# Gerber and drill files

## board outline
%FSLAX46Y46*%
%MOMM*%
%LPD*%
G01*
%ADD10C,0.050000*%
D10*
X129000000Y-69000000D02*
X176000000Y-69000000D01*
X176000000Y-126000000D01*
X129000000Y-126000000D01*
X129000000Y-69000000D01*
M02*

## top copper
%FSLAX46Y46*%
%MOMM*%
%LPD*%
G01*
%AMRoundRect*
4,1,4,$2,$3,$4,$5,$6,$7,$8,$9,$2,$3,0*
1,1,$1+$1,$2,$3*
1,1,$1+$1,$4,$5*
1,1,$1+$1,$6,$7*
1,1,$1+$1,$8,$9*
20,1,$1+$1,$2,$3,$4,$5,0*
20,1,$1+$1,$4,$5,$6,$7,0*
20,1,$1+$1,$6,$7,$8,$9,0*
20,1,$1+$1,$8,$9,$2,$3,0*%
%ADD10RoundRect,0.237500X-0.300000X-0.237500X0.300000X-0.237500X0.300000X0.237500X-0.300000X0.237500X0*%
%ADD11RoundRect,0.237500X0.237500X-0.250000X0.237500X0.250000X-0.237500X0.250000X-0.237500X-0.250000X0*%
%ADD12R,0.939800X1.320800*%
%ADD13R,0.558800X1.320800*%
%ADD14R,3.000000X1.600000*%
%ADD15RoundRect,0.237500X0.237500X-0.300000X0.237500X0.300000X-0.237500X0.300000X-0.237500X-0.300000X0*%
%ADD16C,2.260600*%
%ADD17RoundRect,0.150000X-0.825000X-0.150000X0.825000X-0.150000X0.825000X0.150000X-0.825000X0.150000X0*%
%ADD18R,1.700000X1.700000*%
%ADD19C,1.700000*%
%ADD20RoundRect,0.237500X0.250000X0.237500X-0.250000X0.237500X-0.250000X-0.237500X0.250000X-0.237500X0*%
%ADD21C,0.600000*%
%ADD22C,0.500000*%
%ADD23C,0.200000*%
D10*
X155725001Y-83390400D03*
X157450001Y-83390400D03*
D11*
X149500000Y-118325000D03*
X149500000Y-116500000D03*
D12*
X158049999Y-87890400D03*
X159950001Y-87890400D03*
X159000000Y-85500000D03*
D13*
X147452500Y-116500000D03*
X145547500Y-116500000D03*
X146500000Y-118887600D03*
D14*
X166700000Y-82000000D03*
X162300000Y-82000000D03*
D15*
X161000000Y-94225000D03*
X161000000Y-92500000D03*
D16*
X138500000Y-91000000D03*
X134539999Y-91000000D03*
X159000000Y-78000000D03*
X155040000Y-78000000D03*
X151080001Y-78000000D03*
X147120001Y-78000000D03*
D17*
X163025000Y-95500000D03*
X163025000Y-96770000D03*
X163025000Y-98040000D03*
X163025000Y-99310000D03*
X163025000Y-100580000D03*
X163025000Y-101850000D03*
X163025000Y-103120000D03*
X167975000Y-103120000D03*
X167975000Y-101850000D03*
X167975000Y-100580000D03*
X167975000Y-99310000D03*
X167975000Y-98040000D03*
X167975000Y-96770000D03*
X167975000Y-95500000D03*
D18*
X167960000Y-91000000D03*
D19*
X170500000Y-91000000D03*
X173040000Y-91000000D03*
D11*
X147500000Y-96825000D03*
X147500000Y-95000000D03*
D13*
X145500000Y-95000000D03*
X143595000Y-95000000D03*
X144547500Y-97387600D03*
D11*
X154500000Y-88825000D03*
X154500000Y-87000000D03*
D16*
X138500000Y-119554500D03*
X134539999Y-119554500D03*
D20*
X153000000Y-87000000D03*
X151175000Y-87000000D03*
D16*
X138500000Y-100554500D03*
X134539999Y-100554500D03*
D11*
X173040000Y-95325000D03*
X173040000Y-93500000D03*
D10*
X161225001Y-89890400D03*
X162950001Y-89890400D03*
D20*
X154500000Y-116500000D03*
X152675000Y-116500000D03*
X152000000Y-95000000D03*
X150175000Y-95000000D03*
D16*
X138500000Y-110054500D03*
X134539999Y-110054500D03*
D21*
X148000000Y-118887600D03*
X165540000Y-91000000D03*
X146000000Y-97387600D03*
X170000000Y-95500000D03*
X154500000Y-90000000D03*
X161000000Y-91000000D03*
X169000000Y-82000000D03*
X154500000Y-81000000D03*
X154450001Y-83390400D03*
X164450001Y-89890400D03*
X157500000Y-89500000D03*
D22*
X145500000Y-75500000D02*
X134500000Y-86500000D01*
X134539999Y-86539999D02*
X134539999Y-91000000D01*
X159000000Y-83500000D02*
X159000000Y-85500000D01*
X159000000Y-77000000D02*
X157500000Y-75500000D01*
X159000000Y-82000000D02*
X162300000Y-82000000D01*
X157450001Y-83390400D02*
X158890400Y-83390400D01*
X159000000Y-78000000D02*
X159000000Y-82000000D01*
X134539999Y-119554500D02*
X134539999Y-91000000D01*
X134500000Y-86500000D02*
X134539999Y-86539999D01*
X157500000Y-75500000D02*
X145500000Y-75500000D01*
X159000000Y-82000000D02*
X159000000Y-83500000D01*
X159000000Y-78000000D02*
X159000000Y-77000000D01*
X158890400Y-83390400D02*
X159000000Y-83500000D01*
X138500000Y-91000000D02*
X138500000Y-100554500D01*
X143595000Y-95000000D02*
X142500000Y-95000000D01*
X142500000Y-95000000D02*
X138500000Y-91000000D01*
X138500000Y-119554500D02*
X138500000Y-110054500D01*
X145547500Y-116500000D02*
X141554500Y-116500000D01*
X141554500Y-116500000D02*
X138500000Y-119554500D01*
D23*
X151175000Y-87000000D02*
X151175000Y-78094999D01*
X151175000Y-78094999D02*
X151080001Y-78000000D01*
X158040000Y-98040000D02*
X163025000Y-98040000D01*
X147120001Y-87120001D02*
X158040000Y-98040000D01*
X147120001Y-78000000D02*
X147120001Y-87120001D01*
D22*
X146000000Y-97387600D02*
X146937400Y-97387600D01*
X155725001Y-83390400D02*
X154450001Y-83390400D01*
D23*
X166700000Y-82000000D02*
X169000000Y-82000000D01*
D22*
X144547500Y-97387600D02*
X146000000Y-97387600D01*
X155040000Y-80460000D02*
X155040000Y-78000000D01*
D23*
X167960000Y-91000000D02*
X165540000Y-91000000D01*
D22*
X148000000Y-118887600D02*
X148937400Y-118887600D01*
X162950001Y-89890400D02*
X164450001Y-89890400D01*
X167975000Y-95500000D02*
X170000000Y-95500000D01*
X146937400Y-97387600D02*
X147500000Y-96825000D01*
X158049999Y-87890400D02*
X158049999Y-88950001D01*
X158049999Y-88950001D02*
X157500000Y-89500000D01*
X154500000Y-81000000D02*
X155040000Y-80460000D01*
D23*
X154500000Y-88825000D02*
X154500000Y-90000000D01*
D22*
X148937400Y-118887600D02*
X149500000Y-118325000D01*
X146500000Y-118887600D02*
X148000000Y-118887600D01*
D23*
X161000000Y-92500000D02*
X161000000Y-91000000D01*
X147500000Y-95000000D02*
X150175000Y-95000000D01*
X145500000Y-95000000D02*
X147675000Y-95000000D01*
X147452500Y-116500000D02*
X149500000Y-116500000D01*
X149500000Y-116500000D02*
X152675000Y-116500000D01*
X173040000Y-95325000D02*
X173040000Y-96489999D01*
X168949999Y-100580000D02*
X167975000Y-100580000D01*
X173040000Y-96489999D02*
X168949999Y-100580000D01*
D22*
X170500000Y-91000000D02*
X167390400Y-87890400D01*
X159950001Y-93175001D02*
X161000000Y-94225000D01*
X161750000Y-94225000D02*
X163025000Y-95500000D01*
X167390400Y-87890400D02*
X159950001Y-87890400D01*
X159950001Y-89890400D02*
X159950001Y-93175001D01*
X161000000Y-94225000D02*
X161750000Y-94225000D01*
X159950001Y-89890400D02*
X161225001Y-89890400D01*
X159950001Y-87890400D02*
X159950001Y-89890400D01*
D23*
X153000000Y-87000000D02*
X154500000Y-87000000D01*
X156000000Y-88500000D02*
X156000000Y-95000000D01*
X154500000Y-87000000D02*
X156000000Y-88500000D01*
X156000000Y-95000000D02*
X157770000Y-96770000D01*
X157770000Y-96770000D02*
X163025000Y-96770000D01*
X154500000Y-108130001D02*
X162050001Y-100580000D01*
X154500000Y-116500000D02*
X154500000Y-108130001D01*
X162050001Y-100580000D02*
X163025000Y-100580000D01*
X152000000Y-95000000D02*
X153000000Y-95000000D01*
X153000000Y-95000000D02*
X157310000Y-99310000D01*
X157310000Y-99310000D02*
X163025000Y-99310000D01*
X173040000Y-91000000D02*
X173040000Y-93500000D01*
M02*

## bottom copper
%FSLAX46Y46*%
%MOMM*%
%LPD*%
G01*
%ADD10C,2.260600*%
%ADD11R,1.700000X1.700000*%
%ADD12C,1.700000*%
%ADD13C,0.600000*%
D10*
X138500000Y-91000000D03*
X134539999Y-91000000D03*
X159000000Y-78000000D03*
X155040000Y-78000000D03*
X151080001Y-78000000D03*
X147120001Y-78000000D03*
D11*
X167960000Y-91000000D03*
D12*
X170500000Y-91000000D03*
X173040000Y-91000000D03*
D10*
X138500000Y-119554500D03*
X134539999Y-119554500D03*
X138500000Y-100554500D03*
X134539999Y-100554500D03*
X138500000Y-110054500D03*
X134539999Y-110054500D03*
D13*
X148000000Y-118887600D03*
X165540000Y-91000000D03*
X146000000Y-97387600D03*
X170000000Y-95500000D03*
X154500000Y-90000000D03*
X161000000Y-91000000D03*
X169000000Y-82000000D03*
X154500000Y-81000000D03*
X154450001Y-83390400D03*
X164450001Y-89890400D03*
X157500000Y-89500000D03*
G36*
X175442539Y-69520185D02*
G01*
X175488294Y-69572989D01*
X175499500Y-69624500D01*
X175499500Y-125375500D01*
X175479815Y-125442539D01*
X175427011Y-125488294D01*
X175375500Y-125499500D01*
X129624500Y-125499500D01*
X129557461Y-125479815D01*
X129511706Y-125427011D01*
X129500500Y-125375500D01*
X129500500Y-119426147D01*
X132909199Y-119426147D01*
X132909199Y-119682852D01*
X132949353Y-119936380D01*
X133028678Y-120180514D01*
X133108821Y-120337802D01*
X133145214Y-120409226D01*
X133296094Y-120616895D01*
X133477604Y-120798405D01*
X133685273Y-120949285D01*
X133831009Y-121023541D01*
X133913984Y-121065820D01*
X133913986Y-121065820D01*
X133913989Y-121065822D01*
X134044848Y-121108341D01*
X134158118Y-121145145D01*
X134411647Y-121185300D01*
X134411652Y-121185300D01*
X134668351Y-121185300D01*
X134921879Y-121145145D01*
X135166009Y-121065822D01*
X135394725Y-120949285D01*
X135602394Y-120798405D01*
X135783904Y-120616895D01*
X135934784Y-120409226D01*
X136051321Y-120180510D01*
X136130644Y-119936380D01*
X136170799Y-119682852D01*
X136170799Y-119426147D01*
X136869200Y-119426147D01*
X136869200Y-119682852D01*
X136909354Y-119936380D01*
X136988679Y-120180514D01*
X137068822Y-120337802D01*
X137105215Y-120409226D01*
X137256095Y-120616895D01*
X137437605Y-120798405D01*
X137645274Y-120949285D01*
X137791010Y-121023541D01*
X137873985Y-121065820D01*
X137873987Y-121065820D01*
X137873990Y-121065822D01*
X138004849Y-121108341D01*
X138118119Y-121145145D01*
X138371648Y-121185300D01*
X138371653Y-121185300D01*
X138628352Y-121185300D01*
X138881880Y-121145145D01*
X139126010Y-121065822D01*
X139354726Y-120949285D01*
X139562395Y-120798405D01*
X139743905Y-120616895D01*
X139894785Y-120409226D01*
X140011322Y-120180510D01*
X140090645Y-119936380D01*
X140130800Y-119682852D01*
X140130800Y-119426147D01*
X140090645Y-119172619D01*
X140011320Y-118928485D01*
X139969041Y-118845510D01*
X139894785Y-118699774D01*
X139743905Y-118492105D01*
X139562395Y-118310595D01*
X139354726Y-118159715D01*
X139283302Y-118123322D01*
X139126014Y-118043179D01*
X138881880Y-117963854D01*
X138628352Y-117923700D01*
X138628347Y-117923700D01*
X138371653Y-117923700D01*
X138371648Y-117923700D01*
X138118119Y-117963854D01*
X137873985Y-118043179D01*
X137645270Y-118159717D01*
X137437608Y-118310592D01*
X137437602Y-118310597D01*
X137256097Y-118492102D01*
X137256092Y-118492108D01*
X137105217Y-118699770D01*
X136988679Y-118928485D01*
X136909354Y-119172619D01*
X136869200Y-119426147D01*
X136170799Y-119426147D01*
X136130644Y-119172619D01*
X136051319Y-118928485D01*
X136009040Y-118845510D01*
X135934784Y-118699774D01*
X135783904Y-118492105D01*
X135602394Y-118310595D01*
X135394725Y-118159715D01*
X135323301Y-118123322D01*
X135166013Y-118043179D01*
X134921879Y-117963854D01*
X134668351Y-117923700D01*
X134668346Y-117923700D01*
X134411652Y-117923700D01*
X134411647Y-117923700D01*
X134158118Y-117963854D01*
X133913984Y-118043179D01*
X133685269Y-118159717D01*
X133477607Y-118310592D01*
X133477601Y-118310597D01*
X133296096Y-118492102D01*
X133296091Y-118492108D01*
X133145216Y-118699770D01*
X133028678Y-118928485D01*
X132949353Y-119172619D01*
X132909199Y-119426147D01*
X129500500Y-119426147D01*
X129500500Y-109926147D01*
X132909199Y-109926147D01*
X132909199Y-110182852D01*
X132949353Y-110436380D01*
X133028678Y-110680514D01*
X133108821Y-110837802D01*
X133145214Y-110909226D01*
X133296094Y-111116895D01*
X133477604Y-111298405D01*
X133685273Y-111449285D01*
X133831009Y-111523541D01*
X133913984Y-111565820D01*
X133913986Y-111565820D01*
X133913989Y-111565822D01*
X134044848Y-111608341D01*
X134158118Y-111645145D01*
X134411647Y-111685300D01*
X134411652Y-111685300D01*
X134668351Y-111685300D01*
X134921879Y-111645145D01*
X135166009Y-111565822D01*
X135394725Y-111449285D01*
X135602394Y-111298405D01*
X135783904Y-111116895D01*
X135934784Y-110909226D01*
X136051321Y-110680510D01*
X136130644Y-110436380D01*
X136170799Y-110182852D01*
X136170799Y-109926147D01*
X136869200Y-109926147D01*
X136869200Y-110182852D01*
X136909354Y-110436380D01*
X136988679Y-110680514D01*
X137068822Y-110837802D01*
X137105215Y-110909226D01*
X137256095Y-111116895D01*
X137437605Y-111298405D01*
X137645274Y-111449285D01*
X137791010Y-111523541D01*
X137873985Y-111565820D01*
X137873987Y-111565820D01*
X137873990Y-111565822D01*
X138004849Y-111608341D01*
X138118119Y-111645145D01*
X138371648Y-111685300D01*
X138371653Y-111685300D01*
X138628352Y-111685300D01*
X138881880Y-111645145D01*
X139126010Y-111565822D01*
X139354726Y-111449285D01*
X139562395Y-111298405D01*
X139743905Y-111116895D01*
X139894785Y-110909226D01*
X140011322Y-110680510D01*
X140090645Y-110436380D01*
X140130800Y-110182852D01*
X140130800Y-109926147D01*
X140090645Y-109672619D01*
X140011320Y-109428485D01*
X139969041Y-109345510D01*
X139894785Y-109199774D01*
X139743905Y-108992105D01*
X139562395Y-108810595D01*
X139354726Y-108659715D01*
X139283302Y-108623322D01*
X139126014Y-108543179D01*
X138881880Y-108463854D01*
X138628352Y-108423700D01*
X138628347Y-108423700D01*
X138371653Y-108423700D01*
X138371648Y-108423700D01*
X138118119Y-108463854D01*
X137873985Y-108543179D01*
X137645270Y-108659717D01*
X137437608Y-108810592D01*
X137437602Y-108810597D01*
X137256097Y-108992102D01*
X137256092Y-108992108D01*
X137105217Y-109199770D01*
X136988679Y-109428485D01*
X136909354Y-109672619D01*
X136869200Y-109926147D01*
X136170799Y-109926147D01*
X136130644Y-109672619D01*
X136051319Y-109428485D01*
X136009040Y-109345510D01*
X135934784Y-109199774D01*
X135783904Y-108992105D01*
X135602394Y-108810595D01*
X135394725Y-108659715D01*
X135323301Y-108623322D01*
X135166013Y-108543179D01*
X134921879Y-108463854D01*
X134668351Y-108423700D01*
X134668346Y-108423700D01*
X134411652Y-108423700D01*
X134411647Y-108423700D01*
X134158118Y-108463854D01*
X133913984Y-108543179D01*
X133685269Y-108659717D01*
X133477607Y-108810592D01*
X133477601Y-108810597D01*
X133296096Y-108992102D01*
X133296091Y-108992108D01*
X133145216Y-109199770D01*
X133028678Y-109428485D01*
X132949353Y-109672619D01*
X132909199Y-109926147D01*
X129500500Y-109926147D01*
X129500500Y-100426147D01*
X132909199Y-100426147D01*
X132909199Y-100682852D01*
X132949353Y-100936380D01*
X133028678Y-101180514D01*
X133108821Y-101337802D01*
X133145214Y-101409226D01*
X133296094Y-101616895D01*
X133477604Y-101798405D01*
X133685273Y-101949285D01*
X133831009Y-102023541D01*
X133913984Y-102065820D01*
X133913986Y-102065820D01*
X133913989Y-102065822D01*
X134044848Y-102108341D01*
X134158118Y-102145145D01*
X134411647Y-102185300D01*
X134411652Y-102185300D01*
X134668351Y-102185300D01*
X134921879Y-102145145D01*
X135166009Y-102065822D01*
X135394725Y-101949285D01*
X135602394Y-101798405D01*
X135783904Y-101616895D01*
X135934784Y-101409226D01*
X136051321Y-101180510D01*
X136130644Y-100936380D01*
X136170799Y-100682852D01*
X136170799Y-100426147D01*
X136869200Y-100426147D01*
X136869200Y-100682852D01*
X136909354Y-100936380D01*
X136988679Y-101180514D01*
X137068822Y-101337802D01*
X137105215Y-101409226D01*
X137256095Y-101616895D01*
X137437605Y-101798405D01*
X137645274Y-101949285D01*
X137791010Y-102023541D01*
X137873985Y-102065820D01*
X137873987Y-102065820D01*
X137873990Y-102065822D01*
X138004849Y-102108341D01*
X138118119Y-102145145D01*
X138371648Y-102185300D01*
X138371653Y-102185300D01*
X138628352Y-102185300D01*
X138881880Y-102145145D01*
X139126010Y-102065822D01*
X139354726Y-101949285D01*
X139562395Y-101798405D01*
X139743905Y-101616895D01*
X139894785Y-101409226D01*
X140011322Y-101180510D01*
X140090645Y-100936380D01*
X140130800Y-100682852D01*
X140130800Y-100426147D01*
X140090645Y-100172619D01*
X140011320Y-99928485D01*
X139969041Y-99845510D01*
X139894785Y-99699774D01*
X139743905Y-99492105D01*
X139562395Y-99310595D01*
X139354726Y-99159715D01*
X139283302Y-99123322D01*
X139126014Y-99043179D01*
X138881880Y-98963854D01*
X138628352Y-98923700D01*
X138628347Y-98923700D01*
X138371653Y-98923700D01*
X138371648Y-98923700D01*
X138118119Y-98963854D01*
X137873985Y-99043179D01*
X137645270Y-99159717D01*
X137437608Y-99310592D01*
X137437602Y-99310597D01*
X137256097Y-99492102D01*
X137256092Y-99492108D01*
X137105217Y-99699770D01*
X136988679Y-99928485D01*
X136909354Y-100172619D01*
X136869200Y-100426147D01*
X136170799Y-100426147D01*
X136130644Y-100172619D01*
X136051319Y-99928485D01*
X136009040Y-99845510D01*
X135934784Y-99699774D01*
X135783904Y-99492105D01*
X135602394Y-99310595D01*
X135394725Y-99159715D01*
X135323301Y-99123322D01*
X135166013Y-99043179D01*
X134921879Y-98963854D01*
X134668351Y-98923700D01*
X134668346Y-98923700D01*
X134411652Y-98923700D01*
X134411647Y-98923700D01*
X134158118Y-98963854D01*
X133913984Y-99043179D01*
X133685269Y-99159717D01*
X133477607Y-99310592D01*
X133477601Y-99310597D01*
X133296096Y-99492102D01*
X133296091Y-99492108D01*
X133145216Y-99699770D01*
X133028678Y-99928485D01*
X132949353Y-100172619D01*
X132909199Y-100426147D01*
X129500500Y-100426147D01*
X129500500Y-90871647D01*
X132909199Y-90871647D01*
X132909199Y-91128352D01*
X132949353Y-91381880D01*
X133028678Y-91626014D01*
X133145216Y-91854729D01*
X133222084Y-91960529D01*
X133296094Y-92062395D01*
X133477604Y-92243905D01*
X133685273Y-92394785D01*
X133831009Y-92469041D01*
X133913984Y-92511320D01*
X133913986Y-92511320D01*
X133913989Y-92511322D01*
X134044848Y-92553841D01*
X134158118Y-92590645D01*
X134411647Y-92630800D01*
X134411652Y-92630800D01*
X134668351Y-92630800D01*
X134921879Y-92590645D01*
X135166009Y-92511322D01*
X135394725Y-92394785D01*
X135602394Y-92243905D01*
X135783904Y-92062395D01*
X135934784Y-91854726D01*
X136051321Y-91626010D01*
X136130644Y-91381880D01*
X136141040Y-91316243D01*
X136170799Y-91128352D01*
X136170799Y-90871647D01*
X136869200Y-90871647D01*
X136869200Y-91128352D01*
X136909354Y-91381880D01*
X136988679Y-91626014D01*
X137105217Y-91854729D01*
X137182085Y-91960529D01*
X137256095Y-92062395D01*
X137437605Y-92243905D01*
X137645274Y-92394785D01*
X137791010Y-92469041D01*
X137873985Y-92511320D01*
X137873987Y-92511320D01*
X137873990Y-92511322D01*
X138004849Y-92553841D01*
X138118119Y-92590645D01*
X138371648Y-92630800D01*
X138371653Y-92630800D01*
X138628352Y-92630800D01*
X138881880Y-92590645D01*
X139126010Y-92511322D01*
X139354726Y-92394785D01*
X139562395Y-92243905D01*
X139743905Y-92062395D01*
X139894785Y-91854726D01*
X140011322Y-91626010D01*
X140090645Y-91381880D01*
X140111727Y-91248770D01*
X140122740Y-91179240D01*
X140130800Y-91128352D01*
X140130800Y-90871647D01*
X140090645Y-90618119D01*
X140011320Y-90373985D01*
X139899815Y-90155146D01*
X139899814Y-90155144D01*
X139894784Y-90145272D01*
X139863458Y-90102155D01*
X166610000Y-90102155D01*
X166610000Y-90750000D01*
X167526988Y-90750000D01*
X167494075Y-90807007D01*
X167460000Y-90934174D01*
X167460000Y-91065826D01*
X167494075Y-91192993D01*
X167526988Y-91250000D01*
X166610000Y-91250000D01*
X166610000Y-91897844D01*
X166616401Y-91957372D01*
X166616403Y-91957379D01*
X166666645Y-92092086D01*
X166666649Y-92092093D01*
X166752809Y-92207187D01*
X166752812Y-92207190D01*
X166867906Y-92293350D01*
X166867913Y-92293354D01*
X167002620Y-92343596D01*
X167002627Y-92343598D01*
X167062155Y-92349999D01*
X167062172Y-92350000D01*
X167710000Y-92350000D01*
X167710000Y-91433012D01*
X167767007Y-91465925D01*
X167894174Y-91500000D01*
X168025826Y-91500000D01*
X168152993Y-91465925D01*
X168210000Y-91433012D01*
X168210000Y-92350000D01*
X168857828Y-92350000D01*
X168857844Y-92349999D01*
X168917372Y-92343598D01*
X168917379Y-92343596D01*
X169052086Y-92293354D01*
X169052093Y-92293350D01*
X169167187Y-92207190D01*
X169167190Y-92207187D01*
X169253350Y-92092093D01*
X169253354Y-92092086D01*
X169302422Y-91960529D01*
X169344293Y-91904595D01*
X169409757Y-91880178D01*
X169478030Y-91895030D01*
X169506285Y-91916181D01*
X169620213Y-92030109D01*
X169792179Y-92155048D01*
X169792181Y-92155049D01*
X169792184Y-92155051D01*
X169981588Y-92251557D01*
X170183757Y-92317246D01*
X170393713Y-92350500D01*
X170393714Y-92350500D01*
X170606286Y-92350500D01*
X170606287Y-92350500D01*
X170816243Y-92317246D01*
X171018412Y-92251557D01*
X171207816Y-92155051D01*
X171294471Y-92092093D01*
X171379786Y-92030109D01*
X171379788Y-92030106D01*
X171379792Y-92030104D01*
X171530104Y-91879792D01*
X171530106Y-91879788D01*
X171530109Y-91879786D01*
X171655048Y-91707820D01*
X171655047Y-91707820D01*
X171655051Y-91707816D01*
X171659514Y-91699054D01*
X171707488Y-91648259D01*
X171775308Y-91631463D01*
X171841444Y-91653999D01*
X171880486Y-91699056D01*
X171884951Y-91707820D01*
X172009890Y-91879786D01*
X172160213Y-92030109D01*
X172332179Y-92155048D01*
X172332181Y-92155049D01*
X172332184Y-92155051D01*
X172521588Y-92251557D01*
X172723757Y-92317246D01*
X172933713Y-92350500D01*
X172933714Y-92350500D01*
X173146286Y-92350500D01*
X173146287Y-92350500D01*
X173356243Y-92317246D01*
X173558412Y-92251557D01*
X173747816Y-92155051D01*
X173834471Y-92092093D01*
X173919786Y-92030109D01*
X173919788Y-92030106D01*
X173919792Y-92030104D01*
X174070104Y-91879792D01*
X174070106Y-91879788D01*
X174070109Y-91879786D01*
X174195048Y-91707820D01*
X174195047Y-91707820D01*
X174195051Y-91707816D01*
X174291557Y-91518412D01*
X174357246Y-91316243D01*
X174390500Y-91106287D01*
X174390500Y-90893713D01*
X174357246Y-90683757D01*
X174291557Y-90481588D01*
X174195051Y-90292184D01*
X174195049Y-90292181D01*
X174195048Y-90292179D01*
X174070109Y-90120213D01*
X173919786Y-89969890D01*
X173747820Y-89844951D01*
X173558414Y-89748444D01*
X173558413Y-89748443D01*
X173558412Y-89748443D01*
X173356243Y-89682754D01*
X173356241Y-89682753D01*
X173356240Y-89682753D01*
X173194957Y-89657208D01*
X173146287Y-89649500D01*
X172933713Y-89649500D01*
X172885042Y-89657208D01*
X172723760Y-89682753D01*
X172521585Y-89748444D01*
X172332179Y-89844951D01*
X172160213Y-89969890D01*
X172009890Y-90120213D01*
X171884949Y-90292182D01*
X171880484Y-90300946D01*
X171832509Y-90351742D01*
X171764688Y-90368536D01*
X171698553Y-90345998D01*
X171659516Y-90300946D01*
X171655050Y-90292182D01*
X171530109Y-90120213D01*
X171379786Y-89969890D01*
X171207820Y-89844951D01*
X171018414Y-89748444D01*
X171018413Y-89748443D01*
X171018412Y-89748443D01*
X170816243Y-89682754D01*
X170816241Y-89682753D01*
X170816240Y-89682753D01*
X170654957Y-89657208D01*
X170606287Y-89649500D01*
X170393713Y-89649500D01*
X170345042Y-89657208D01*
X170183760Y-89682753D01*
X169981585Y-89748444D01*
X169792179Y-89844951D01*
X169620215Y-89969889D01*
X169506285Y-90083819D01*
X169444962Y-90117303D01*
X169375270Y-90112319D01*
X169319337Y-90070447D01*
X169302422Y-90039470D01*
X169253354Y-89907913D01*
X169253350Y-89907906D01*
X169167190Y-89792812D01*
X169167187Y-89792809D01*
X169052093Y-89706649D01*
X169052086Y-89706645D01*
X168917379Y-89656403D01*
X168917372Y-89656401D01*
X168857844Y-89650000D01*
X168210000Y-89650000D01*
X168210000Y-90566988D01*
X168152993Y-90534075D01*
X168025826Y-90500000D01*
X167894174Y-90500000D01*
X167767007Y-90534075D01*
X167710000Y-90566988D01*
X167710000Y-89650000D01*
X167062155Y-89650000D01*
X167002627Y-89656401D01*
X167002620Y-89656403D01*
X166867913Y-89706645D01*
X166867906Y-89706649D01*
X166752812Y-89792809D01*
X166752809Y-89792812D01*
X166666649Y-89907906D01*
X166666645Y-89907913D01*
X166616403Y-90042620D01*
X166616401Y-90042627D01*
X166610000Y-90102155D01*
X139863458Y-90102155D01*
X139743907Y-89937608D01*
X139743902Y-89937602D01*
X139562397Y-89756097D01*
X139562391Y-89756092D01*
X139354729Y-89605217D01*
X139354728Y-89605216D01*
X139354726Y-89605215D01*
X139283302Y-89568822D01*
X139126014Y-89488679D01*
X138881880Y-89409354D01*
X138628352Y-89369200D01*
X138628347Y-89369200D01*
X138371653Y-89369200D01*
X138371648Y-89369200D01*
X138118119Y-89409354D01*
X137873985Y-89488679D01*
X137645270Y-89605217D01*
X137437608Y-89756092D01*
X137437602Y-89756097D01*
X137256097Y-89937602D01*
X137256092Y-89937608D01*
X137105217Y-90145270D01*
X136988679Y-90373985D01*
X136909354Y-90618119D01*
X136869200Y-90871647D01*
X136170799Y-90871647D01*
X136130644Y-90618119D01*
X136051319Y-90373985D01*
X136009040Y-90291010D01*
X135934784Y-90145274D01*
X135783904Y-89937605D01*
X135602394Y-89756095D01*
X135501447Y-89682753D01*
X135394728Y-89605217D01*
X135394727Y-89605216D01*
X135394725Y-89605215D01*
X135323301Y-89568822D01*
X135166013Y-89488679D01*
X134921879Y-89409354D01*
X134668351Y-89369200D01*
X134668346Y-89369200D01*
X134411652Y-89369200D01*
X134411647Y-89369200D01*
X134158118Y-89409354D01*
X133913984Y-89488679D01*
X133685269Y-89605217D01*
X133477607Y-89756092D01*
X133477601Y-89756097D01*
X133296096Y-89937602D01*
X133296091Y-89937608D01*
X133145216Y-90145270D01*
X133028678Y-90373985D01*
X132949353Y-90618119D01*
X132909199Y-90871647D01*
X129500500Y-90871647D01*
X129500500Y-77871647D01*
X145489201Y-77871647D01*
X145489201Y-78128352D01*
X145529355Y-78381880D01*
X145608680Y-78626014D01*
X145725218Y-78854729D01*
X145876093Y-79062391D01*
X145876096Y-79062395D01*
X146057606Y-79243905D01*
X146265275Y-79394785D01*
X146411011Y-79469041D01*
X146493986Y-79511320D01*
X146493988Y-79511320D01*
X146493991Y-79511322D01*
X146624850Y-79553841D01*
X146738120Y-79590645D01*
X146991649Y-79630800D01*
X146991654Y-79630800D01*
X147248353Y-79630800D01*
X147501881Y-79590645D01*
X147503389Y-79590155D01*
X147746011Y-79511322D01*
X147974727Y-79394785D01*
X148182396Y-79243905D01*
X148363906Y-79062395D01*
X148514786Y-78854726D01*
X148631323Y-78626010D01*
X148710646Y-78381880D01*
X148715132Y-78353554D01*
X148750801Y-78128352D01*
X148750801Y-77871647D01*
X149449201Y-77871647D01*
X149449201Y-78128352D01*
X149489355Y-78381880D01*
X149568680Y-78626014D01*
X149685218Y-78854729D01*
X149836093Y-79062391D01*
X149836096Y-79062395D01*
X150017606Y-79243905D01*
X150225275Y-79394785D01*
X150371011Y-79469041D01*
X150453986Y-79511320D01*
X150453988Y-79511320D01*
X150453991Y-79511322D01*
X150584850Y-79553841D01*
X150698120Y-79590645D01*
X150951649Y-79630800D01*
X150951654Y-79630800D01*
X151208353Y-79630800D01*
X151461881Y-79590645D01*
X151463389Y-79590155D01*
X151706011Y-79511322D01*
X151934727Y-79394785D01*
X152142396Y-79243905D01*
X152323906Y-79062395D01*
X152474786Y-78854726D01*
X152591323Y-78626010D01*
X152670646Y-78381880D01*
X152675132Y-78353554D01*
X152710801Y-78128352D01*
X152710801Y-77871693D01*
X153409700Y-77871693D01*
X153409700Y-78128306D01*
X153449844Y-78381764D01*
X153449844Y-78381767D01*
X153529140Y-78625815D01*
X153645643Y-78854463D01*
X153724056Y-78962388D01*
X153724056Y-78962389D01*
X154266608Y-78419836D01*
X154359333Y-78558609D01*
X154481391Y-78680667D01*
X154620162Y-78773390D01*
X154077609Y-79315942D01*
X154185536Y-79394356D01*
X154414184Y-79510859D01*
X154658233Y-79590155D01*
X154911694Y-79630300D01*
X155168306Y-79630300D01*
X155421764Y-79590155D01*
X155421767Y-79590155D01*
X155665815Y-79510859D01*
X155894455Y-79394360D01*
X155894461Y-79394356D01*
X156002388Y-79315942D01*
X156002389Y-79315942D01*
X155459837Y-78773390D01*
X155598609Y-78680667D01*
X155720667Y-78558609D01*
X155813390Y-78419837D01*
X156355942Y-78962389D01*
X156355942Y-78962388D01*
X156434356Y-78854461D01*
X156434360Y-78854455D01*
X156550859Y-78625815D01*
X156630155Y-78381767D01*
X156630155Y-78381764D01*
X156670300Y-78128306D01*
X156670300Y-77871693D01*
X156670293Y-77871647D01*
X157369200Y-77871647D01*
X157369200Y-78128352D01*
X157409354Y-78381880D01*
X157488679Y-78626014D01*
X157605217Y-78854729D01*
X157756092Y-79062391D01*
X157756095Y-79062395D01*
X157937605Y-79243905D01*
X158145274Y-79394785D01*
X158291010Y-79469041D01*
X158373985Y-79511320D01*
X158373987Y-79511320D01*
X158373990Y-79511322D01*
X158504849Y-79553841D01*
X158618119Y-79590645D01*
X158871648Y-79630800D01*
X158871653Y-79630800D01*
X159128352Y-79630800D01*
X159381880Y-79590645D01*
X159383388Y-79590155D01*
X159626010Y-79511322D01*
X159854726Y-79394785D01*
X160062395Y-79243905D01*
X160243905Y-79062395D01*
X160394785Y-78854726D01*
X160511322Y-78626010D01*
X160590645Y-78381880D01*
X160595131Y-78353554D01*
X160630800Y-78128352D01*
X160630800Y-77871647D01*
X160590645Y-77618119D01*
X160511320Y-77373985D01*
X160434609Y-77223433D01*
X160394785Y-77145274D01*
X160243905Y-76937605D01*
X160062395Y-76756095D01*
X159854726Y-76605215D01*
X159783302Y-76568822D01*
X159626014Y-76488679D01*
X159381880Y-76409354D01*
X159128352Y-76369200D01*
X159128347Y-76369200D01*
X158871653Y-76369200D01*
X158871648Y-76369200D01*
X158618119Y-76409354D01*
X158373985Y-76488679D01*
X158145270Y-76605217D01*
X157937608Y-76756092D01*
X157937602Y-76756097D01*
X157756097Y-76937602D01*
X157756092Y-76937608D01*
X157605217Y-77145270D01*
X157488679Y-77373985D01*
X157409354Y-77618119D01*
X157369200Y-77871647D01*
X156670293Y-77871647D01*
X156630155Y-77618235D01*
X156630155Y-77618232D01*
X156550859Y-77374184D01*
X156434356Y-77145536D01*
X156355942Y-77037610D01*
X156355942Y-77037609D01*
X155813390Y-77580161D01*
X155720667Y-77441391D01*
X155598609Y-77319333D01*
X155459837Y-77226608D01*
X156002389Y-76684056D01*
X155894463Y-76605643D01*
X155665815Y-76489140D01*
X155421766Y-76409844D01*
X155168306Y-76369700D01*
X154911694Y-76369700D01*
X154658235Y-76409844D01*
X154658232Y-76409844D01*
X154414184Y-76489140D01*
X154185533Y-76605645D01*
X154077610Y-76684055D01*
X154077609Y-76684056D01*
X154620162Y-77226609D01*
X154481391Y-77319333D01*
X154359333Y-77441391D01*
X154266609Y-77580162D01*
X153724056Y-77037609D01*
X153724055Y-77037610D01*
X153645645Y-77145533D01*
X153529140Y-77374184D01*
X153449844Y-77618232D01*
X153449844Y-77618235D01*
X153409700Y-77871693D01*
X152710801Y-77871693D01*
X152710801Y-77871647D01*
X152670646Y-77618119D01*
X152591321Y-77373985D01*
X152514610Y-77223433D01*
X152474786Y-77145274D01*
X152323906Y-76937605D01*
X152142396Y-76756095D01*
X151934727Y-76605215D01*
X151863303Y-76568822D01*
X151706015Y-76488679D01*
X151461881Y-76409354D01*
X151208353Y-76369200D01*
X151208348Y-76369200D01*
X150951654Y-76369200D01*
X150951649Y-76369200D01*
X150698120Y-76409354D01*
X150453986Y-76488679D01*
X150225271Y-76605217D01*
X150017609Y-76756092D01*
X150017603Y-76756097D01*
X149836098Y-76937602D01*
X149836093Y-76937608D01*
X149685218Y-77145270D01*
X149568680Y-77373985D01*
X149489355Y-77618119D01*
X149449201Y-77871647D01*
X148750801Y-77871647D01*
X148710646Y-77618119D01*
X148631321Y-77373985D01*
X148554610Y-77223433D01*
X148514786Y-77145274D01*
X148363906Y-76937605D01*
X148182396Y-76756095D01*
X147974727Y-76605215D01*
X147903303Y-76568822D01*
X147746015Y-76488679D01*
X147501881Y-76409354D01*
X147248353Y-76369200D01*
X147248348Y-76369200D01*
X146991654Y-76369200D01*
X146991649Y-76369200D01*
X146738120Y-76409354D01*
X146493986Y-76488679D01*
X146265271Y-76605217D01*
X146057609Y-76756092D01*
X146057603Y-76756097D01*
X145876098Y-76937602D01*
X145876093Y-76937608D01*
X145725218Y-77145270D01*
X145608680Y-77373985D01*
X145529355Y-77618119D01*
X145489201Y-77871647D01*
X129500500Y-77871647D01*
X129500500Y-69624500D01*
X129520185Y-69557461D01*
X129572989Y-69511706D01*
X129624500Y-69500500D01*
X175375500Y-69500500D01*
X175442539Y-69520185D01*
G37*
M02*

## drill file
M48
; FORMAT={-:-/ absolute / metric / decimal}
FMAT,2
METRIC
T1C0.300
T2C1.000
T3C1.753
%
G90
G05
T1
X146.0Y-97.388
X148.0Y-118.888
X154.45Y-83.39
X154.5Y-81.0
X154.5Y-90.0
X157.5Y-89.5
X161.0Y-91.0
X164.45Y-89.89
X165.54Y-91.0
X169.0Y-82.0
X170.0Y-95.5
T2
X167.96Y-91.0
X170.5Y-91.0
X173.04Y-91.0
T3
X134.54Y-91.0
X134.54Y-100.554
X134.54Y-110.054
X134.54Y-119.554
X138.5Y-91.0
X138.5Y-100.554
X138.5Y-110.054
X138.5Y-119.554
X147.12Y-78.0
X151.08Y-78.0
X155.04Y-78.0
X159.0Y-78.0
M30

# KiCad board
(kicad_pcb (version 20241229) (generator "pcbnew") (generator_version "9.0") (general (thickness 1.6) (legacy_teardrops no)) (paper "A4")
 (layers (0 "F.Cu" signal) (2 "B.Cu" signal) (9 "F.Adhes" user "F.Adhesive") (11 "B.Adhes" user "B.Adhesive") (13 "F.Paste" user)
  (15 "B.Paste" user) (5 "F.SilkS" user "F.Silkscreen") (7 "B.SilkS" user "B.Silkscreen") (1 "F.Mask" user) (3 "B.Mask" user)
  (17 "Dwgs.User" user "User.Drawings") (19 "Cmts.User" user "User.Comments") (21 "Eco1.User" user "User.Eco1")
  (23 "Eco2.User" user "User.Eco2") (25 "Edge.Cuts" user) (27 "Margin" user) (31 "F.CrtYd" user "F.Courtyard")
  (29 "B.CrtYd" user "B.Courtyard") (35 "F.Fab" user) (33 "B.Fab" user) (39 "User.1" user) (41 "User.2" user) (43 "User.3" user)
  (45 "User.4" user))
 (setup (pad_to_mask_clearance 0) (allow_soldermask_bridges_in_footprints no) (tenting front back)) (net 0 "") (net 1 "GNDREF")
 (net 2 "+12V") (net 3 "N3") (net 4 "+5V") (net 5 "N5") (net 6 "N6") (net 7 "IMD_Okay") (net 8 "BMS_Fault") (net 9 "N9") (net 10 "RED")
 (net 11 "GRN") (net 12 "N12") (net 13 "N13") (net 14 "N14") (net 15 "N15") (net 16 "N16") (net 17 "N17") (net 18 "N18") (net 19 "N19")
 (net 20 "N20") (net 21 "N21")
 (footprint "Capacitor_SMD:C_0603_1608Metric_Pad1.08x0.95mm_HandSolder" (layer "F.Cu") (at 156.587501 83.3904)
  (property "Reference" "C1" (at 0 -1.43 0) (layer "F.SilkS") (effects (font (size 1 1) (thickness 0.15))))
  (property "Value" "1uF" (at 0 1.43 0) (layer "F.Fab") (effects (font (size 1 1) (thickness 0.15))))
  (pad "1" smd roundrect (at -0.8625 0) (size 1.075 0.95) (layers "F.Cu" "F.Mask" "F.Paste") (roundrect_rratio 0.25) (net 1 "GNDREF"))
  (pad "2" smd roundrect (at 0.8625 0) (size 1.075 0.95) (layers "F.Cu" "F.Mask" "F.Paste") (roundrect_rratio 0.25) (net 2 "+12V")))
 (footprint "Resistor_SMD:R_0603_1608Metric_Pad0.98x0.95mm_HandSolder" (layer "F.Cu") (at 149.5 117.4125 90)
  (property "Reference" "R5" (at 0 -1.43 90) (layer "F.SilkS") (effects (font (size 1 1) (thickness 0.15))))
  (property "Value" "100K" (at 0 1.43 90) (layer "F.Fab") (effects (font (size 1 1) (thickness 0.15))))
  (pad "1" smd roundrect (at -0.9125 0 90) (size 0.975 0.95) (layers "F.Cu" "F.Mask" "F.Paste") (roundrect_rratio 0.25) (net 1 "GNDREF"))
  (pad "2" smd roundrect (at 0.9125 0 90) (size 0.975 0.95) (layers "F.Cu" "F.Mask" "F.Paste") (roundrect_rratio 0.25) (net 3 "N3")))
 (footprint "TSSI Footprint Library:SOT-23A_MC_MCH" (layer "F.Cu") (at 159 86.6952)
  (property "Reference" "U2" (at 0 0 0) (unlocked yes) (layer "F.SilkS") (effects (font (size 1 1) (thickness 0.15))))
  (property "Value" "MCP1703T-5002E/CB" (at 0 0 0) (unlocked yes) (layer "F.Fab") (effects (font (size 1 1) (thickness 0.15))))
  (pad "1" smd rect (at -0.950001 1.1952) (size 0.9398 1.3208) (layers "F.Cu" "F.Mask" "F.Paste") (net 1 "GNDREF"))
  (pad "2" smd rect (at 0.950001 1.1952) (size 0.9398 1.3208) (layers "F.Cu" "F.Mask" "F.Paste") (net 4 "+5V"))
  (pad "3" smd rect (at 0 -1.1952) (size 0.9398 1.3208) (layers "F.Cu" "F.Mask" "F.Paste") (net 2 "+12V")))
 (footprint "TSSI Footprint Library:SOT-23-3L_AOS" (layer "F.Cu") (at 146.5 117.6938 180)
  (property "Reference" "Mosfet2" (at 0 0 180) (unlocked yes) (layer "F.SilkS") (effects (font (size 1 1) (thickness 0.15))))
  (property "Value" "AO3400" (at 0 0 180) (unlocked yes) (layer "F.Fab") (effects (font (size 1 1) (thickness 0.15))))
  (pad "1" smd rect (at -0.9525 1.1938 180) (size 0.5588 1.3208) (layers "F.Cu" "F.Mask" "F.Paste") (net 3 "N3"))
  (pad "2" smd rect (at 0.9525 1.1938 180) (size 0.5588 1.3208) (layers "F.Cu" "F.Mask" "F.Paste") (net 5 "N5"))
  (pad "3" smd rect (at 0 -1.1938 180) (size 0.5588 1.3208) (layers "F.Cu" "F.Mask" "F.Paste") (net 1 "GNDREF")))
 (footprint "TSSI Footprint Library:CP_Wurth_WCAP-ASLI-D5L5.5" (layer "F.Cu") (at 164.5 82 180)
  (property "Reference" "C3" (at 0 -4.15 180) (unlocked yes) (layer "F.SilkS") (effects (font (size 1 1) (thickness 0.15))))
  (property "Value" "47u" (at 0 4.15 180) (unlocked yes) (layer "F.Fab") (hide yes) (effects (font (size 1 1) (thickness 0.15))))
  (pad "1" smd rect (at -2.2 0 180) (size 3 1.6) (layers "F.Cu" "F.Mask" "F.Paste") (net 1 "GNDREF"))
  (pad "2" smd rect (at 2.2 0 180) (size 3 1.6) (layers "F.Cu" "F.Mask" "F.Paste") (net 2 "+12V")))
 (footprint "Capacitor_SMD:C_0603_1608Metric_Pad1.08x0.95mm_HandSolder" (layer "F.Cu") (at 161 93.3625 90)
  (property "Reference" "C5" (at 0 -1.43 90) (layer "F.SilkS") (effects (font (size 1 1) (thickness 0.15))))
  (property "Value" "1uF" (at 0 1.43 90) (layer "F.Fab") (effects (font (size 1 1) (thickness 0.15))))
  (pad "1" smd roundrect (at -0.8625 0 90) (size 1.075 0.95) (layers "F.Cu" "F.Mask" "F.Paste") (roundrect_rratio 0.25) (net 4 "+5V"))
  (pad "2" smd roundrect (at 0.8625 0 90) (size 1.075 0.95) (layers "F.Cu" "F.Mask" "F.Paste") (roundrect_rratio 0.25) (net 1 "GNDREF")))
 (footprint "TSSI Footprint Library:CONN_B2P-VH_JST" (layer "F.Cu") (at 138.5 91 180)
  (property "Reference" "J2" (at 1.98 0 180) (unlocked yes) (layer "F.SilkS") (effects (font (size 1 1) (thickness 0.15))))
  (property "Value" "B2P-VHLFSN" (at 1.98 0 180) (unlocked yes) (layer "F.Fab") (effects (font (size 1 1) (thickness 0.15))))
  (pad "1" thru_hole circle (at 0 0 180) (size 2.2606 2.2606) (drill 1.7526) (layers "*.Cu" "*.Mask") (remove_unused_layers no) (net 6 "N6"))
  (pad "2" thru_hole circle (at 3.960001 0 180) (size 2.2606 2.2606) (drill 1.7526) (layers "*.Cu" "*.Mask") (remove_unused_layers no)
   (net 2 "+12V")))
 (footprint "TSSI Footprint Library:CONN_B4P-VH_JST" (layer "F.Cu") (at 159 78 180)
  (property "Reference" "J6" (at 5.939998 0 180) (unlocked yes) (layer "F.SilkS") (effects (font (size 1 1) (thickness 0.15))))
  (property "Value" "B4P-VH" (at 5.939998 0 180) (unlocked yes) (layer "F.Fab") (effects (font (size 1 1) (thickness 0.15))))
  (pad "1" thru_hole circle (at 0 0 180) (size 2.2606 2.2606) (drill 1.7526) (layers "*.Cu" "*.Mask") (remove_unused_layers no)
   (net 2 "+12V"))
  (pad "2" thru_hole circle (at 3.96 0 180) (size 2.2606 2.2606) (drill 1.7526) (layers "*.Cu" "*.Mask") (remove_unused_layers no)
   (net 1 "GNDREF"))
  (pad "3" thru_hole circle (at 7.919999 0 180) (size 2.2606 2.2606) (drill 1.7526) (layers "*.Cu" "*.Mask") (remove_unused_layers no)
   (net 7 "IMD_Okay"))
  (pad "4" thru_hole circle (at 11.879999 0 180) (size 2.2606 2.2606) (drill 1.7526) (layers "*.Cu" "*.Mask") (remove_unused_layers no)
   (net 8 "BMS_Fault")))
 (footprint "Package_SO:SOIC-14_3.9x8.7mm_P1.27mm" (layer "F.Cu") (at 165.5 99.31)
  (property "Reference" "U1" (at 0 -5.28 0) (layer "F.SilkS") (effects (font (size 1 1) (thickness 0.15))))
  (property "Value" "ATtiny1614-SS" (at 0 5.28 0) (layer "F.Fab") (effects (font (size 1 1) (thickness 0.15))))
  (pad "1" smd roundrect (at -2.475 -3.81) (size 1.95 0.6) (layers "F.Cu" "F.Mask" "F.Paste") (roundrect_rratio 0.25) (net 4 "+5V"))
  (pad "2" smd roundrect (at -2.475 -2.54) (size 1.95 0.6) (layers "F.Cu" "F.Mask" "F.Paste") (roundrect_rratio 0.25) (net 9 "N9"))
  (pad "3" smd roundrect (at -2.475 -1.27) (size 1.95 0.6) (layers "F.Cu" "F.Mask" "F.Paste") (roundrect_rratio 0.25) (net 8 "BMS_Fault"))
  (pad "4" smd roundrect (at -2.475 0) (size 1.95 0.6) (layers "F.Cu" "F.Mask" "F.Paste") (roundrect_rratio 0.25) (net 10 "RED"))
  (pad "5" smd roundrect (at -2.475 1.27) (size 1.95 0.6) (layers "F.Cu" "F.Mask" "F.Paste") (roundrect_rratio 0.25) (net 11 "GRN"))
  (pad "6" smd roundrect (at -2.475 2.54) (size 1.95 0.6) (layers "F.Cu" "F.Mask" "F.Paste") (roundrect_rratio 0.25) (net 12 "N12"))
  (pad "7" smd roundrect (at -2.475 3.81) (size 1.95 0.6) (layers "F.Cu" "F.Mask" "F.Paste") (roundrect_rratio 0.25) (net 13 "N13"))
  (pad "8" smd roundrect (at 2.475 3.81) (size 1.95 0.6) (layers "F.Cu" "F.Mask" "F.Paste") (roundrect_rratio 0.25) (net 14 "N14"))
  (pad "9" smd roundrect (at 2.475 2.54) (size 1.95 0.6) (layers "F.Cu" "F.Mask" "F.Paste") (roundrect_rratio 0.25) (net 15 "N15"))
  (pad "10" smd roundrect (at 2.475 1.27) (size 1.95 0.6) (layers "F.Cu" "F.Mask" "F.Paste") (roundrect_rratio 0.25) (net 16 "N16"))
  (pad "11" smd roundrect (at 2.475 0) (size 1.95 0.6) (layers "F.Cu" "F.Mask" "F.Paste") (roundrect_rratio 0.25) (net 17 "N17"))
  (pad "12" smd roundrect (at 2.475 -1.27) (size 1.95 0.6) (layers "F.Cu" "F.Mask" "F.Paste") (roundrect_rratio 0.25) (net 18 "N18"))
  (pad "13" smd roundrect (at 2.475 -2.54) (size 1.95 0.6) (layers "F.Cu" "F.Mask" "F.Paste") (roundrect_rratio 0.25) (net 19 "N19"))
  (pad "14" smd roundrect (at 2.475 -3.81) (size 1.95 0.6) (layers "F.Cu" "F.Mask" "F.Paste") (roundrect_rratio 0.25) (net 1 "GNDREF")))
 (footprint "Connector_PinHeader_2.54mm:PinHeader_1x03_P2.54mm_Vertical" (layer "F.Cu") (at 167.96 91 90)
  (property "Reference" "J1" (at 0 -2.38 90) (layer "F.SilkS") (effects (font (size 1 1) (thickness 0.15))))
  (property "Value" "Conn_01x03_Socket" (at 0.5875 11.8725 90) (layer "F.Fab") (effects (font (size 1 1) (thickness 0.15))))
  (pad "1" thru_hole rect (at 0 0 90) (size 1.7 1.7) (drill 1) (layers "*.Cu" "*.Mask") (remove_unused_layers no) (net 1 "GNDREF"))
  (pad "2" thru_hole circle (at 0 2.54 90) (size 1.7 1.7) (drill 1) (layers "*.Cu" "*.Mask") (remove_unused_layers no) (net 4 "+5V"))
  (pad "3" thru_hole circle (at 0 5.08 90) (size 1.7 1.7) (drill 1) (layers "*.Cu" "*.Mask") (remove_unused_layers no) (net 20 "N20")))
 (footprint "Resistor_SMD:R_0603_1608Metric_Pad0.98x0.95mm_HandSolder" (layer "F.Cu") (at 147.5 95.9125 90)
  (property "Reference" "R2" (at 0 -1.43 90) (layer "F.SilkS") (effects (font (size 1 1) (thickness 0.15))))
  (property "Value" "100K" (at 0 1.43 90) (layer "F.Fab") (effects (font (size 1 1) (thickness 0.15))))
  (pad "1" smd roundrect (at -0.9125 0 90) (size 0.975 0.95) (layers "F.Cu" "F.Mask" "F.Paste") (roundrect_rratio 0.25) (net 1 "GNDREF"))
  (pad "2" smd roundrect (at 0.9125 0 90) (size 0.975 0.95) (layers "F.Cu" "F.Mask" "F.Paste") (roundrect_rratio 0.25) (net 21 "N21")))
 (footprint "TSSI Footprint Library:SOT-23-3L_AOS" (layer "F.Cu") (at 144.5475 96.1938 180)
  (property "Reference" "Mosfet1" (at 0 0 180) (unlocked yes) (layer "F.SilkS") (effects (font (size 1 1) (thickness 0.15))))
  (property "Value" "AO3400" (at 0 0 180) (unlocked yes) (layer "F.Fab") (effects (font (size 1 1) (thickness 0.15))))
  (pad "1" smd rect (at -0.9525 1.1938 180) (size 0.5588 1.3208) (layers "F.Cu" "F.Mask" "F.Paste") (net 21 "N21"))
  (pad "2" smd rect (at 0.9525 1.1938 180) (size 0.5588 1.3208) (layers "F.Cu" "F.Mask" "F.Paste") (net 6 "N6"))
  (pad "3" smd rect (at 0 -1.1938 180) (size 0.5588 1.3208) (layers "F.Cu" "F.Mask" "F.Paste") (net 1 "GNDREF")))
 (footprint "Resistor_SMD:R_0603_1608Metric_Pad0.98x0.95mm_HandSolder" (layer "F.Cu") (at 154.5 87.9125 90)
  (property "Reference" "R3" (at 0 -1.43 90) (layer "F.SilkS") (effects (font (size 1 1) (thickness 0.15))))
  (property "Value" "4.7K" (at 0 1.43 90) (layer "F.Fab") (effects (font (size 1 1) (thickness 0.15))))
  (pad "1" smd roundrect (at -0.9125 0 90) (size 0.975 0.95) (layers "F.Cu" "F.Mask" "F.Paste") (roundrect_rratio 0.25) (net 1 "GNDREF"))
  (pad "2" smd roundrect (at 0.9125 0 90) (size 0.975 0.95) (layers "F.Cu" "F.Mask" "F.Paste") (roundrect_rratio 0.25) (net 9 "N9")))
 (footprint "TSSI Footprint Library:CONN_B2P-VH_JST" (layer "F.Cu") (at 138.5 119.5545 180)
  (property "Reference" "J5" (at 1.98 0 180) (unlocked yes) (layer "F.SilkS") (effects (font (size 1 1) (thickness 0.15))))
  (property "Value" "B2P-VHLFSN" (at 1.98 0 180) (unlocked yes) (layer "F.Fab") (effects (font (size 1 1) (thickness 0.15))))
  (pad "1" thru_hole circle (at 0 0 180) (size 2.2606 2.2606) (drill 1.7526) (layers "*.Cu" "*.Mask") (remove_unused_layers no) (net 5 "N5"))
  (pad "2" thru_hole circle (at 3.960001 0 180) (size 2.2606 2.2606) (drill 1.7526) (layers "*.Cu" "*.Mask") (remove_unused_layers no)
   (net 2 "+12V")))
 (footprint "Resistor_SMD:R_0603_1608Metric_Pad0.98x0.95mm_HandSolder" (layer "F.Cu") (at 152.0875 87 180)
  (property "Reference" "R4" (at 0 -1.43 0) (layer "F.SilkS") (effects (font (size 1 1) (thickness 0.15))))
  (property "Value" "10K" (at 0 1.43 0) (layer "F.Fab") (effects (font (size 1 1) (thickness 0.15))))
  (pad "1" smd roundrect (at -0.9125 0 180) (size 0.975 0.95) (layers "F.Cu" "F.Mask" "F.Paste") (roundrect_rratio 0.25) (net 9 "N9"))
  (pad "2" smd roundrect (at 0.9125 0 180) (size 0.975 0.95) (layers "F.Cu" "F.Mask" "F.Paste") (roundrect_rratio 0.25) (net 7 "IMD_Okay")))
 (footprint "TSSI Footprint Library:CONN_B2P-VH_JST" (layer "F.Cu") (at 138.5 100.5545 180)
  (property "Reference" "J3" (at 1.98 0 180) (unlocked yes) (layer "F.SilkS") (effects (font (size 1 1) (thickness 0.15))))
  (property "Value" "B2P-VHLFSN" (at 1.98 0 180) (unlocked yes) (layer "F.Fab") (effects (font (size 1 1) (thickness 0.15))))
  (pad "1" thru_hole circle (at 0 0 180) (size 2.2606 2.2606) (drill 1.7526) (layers "*.Cu" "*.Mask") (remove_unused_layers no) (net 6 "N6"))
  (pad "2" thru_hole circle (at 3.960001 0 180) (size 2.2606 2.2606) (drill 1.7526) (layers "*.Cu" "*.Mask") (remove_unused_layers no)
   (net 2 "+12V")))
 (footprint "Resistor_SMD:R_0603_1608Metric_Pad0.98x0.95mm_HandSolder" (layer "F.Cu") (at 173.04 94.4125 90)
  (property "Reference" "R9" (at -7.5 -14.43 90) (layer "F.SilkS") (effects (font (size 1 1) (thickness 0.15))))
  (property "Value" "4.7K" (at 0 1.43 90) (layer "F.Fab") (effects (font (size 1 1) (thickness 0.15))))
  (pad "1" smd roundrect (at -0.9125 0 90) (size 0.975 0.95) (layers "F.Cu" "F.Mask" "F.Paste") (roundrect_rratio 0.25) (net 16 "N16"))
  (pad "2" smd roundrect (at 0.9125 0 90) (size 0.975 0.95) (layers "F.Cu" "F.Mask" "F.Paste") (roundrect_rratio 0.25) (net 20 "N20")))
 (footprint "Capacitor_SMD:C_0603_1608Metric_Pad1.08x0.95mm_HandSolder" (layer "F.Cu") (at 162.087501 89.8904)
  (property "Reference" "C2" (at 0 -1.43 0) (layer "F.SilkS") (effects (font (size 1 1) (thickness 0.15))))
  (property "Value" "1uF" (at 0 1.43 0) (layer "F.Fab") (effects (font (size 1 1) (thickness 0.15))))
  (pad "1" smd roundrect (at -0.8625 0) (size 1.075 0.95) (layers "F.Cu" "F.Mask" "F.Paste") (roundrect_rratio 0.25) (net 4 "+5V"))
  (pad "2" smd roundrect (at 0.8625 0) (size 1.075 0.95) (layers "F.Cu" "F.Mask" "F.Paste") (roundrect_rratio 0.25) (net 1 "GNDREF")))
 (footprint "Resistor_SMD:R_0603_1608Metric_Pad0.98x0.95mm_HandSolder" (layer "F.Cu") (at 153.5875 116.5 180)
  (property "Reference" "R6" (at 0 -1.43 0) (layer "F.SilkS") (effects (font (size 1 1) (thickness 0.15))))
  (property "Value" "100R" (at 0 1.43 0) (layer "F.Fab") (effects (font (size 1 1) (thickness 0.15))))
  (pad "1" smd roundrect (at -0.9125 0 180) (size 0.975 0.95) (layers "F.Cu" "F.Mask" "F.Paste") (roundrect_rratio 0.25) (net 11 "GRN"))
  (pad "2" smd roundrect (at 0.9125 0 180) (size 0.975 0.95) (layers "F.Cu" "F.Mask" "F.Paste") (roundrect_rratio 0.25) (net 3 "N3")))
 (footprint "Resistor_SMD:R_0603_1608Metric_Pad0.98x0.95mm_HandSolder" (layer "F.Cu") (at 151.0875 95 180)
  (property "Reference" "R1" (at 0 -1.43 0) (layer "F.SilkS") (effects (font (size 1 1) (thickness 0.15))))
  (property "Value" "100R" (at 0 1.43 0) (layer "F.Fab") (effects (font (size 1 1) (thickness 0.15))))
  (pad "1" smd roundrect (at -0.9125 0 180) (size 0.975 0.95) (layers "F.Cu" "F.Mask" "F.Paste") (roundrect_rratio 0.25) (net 10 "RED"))
  (pad "2" smd roundrect (at 0.9125 0 180) (size 0.975 0.95) (layers "F.Cu" "F.Mask" "F.Paste") (roundrect_rratio 0.25) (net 21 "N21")))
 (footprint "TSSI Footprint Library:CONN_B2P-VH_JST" (layer "F.Cu") (at 138.5 110.0545 180)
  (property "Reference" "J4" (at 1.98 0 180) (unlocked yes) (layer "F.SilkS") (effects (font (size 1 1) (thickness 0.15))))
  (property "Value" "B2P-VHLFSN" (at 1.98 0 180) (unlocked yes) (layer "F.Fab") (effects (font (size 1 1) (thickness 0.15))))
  (pad "1" thru_hole circle (at 0 0 180) (size 2.2606 2.2606) (drill 1.7526) (layers "*.Cu" "*.Mask") (remove_unused_layers no) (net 5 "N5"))
  (pad "2" thru_hole circle (at 3.960001 0 180) (size 2.2606 2.2606) (drill 1.7526) (layers "*.Cu" "*.Mask") (remove_unused_layers no)
   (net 2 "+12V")))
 (gr_rect (start 129 69) (end 176 126) (stroke (width 0.05) (type default)) (fill no) (layer "Edge.Cuts"))
 (segment (start 145.5 75.5) (end 134.5 86.5) (width 0.5) (layer "F.Cu") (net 2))
 (segment (start 134.539999 86.539999) (end 134.539999 91) (width 0.5) (layer "F.Cu") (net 2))
 (segment (start 159 83.5) (end 159 85.5) (width 0.5) (layer "F.Cu") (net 2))
 (segment (start 159 77) (end 157.5 75.5) (width 0.5) (layer "F.Cu") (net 2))
 (segment (start 159 82) (end 162.3 82) (width 0.5) (layer "F.Cu") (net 2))
 (segment (start 157.450001 83.3904) (end 158.8904 83.3904) (width 0.5) (layer "F.Cu") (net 2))
 (segment (start 159 78) (end 159 82) (width 0.5) (layer "F.Cu") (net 2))
 (segment (start 134.539999 119.5545) (end 134.539999 91) (width 0.5) (layer "F.Cu") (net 2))
 (segment (start 134.5 86.5) (end 134.539999 86.539999) (width 0.5) (layer "F.Cu") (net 2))
 (segment (start 157.5 75.5) (end 145.5 75.5) (width 0.5) (layer "F.Cu") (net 2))
 (segment (start 159 82) (end 159 83.5) (width 0.5) (layer "F.Cu") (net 2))
 (segment (start 159 78) (end 159 77) (width 0.5) (layer "F.Cu") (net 2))
 (segment (start 158.8904 83.3904) (end 159 83.5) (width 0.5) (layer "F.Cu") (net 2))
 (segment (start 138.5 91) (end 138.5 100.5545) (width 0.5) (layer "F.Cu") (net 6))
 (segment (start 143.595 95) (end 142.5 95) (width 0.5) (layer "F.Cu") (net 6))
 (segment (start 142.5 95) (end 138.5 91) (width 0.5) (layer "F.Cu") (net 6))
 (segment (start 138.5 119.5545) (end 138.5 110.0545) (width 0.5) (layer "F.Cu") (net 5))
 (segment (start 145.5475 116.5) (end 141.5545 116.5) (width 0.5) (layer "F.Cu") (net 5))
 (segment (start 141.5545 116.5) (end 138.5 119.5545) (width 0.5) (layer "F.Cu") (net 5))
 (segment (start 151.175 87) (end 151.175 78.094999) (width 0.2) (layer "F.Cu") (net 7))
 (segment (start 151.175 78.094999) (end 151.080001 78) (width 0.2) (layer "F.Cu") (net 7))
 (segment (start 158.04 98.04) (end 163.025 98.04) (width 0.2) (layer "F.Cu") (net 8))
 (segment (start 147.120001 87.120001) (end 158.04 98.04) (width 0.2) (layer "F.Cu") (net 8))
 (segment (start 147.120001 78) (end 147.120001 87.120001) (width 0.2) (layer "F.Cu") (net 8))
 (segment (start 146 97.3876) (end 146.9374 97.3876) (width 0.5) (layer "F.Cu") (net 1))
 (segment (start 155.725001 83.3904) (end 154.450001 83.3904) (width 0.5) (layer "F.Cu") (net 1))
 (segment (start 166.7 82) (end 169 82) (width 0.2) (layer "F.Cu") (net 1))
 (segment (start 144.5475 97.3876) (end 146 97.3876) (width 0.5) (layer "F.Cu") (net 1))
 (segment (start 155.04 80.46) (end 155.04 78) (width 0.5) (layer "F.Cu") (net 1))
 (segment (start 167.96 91) (end 165.54 91) (width 0.2) (layer "F.Cu") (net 1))
 (segment (start 148 118.8876) (end 148.9374 118.8876) (width 0.5) (layer "F.Cu") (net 1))
 (segment (start 162.950001 89.8904) (end 164.450001 89.8904) (width 0.5) (layer "F.Cu") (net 1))
 (segment (start 167.975 95.5) (end 170 95.5) (width 0.5) (layer "F.Cu") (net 1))
 (segment (start 146.9374 97.3876) (end 147.5 96.825) (width 0.5) (layer "F.Cu") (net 1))
 (segment (start 158.049999 87.8904) (end 158.049999 88.950001) (width 0.5) (layer "F.Cu") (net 1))
 (segment (start 158.049999 88.950001) (end 157.5 89.5) (width 0.5) (layer "F.Cu") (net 1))
 (segment (start 154.5 81) (end 155.04 80.46) (width 0.5) (layer "F.Cu") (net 1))
 (segment (start 154.5 88.825) (end 154.5 90) (width 0.2) (layer "F.Cu") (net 1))
 (segment (start 148.9374 118.8876) (end 149.5 118.325) (width 0.5) (layer "F.Cu") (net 1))
 (segment (start 146.5 118.8876) (end 148 118.8876) (width 0.5) (layer "F.Cu") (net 1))
 (segment (start 161 92.5) (end 161 91) (width 0.2) (layer "F.Cu") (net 1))
 (via (at 148 118.8876) (size 0.6) (drill 0.3) (layers "F.Cu" "B.Cu") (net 1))
 (via (at 165.54 91) (size 0.6) (drill 0.3) (layers "F.Cu" "B.Cu") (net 1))
 (via (at 146 97.3876) (size 0.6) (drill 0.3) (layers "F.Cu" "B.Cu") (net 1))
 (via (at 170 95.5) (size 0.6) (drill 0.3) (layers "F.Cu" "B.Cu") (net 1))
 (via (at 154.5 90) (size 0.6) (drill 0.3) (layers "F.Cu" "B.Cu") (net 1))
 (via (at 161 91) (size 0.6) (drill 0.3) (layers "F.Cu" "B.Cu") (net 1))
 (via (at 169 82) (size 0.6) (drill 0.3) (layers "F.Cu" "B.Cu") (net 1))
 (via (at 154.5 81) (size 0.6) (drill 0.3) (layers "F.Cu" "B.Cu") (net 1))
 (via (at 154.450001 83.3904) (size 0.6) (drill 0.3) (layers "F.Cu" "B.Cu") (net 1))
 (via (at 164.450001 89.8904) (size 0.6) (drill 0.3) (layers "F.Cu" "B.Cu") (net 1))
 (via (at 157.5 89.5) (size 0.6) (drill 0.3) (layers "F.Cu" "B.Cu") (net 1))
 (segment (start 147.5 95) (end 150.175 95) (width 0.2) (layer "F.Cu") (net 21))
 (segment (start 145.5 95) (end 147.675 95) (width 0.2) (layer "F.Cu") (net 21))
 (segment (start 147.4525 116.5) (end 149.5 116.5) (width 0.2) (layer "F.Cu") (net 3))
 (segment (start 149.5 116.5) (end 152.675 116.5) (width 0.2) (layer "F.Cu") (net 3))
 (segment (start 173.04 95.325) (end 173.04 96.489999) (width 0.2) (layer "F.Cu") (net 16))
 (segment (start 168.949999 100.58) (end 167.975 100.58) (width 0.2) (layer "F.Cu") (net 16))
 (segment (start 173.04 96.489999) (end 168.949999 100.58) (width 0.2) (layer "F.Cu") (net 16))
 (segment (start 170.5 91) (end 167.3904 87.8904) (width 0.5) (layer "F.Cu") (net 4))
 (segment (start 159.950001 93.175001) (end 161 94.225) (width 0.5) (layer "F.Cu") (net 4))
 (segment (start 161.75 94.225) (end 163.025 95.5) (width 0.5) (layer "F.Cu") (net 4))
 (segment (start 167.3904 87.8904) (end 159.950001 87.8904) (width 0.5) (layer "F.Cu") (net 4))
 (segment (start 159.950001 89.8904) (end 159.950001 93.175001) (width 0.5) (layer "F.Cu") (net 4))
 (segment (start 161 94.225) (end 161.75 94.225) (width 0.5) (layer "F.Cu") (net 4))
 (segment (start 159.950001 89.8904) (end 161.225001 89.8904) (width 0.5) (layer "F.Cu") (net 4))
 (segment (start 159.950001 87.8904) (end 159.950001 89.8904) (width 0.5) (layer "F.Cu") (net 4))
 (segment (start 153 87) (end 154.5 87) (width 0.2) (layer "F.Cu") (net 9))
 (segment (start 156 88.5) (end 156 95) (width 0.2) (layer "F.Cu") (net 9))
 (segment (start 154.5 87) (end 156 88.5) (width 0.2) (layer "F.Cu") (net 9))
 (segment (start 156 95) (end 157.77 96.77) (width 0.2) (layer "F.Cu") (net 9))
 (segment (start 157.77 96.77) (end 163.025 96.77) (width 0.2) (layer "F.Cu") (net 9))
 (segment (start 154.5 108.130001) (end 162.050001 100.58) (width 0.2) (layer "F.Cu") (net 11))
 (segment (start 154.5 116.5) (end 154.5 108.130001) (width 0.2) (layer "F.Cu") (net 11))
 (segment (start 162.050001 100.58) (end 163.025 100.58) (width 0.2) (layer "F.Cu") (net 11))
 (segment (start 152 95) (end 153 95) (width 0.2) (layer "F.Cu") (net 10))
 (segment (start 153 95) (end 157.31 99.31) (width 0.2) (layer "F.Cu") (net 10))
 (segment (start 157.31 99.31) (end 163.025 99.31) (width 0.2) (layer "F.Cu") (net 10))
 (segment (start 173.04 91) (end 173.04 93.5) (width 0.2) (layer "F.Cu") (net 20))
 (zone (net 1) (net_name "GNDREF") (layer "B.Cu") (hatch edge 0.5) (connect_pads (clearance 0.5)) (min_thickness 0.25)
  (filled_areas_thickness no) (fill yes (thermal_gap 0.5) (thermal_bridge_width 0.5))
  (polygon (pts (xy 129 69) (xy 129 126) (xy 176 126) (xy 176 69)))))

